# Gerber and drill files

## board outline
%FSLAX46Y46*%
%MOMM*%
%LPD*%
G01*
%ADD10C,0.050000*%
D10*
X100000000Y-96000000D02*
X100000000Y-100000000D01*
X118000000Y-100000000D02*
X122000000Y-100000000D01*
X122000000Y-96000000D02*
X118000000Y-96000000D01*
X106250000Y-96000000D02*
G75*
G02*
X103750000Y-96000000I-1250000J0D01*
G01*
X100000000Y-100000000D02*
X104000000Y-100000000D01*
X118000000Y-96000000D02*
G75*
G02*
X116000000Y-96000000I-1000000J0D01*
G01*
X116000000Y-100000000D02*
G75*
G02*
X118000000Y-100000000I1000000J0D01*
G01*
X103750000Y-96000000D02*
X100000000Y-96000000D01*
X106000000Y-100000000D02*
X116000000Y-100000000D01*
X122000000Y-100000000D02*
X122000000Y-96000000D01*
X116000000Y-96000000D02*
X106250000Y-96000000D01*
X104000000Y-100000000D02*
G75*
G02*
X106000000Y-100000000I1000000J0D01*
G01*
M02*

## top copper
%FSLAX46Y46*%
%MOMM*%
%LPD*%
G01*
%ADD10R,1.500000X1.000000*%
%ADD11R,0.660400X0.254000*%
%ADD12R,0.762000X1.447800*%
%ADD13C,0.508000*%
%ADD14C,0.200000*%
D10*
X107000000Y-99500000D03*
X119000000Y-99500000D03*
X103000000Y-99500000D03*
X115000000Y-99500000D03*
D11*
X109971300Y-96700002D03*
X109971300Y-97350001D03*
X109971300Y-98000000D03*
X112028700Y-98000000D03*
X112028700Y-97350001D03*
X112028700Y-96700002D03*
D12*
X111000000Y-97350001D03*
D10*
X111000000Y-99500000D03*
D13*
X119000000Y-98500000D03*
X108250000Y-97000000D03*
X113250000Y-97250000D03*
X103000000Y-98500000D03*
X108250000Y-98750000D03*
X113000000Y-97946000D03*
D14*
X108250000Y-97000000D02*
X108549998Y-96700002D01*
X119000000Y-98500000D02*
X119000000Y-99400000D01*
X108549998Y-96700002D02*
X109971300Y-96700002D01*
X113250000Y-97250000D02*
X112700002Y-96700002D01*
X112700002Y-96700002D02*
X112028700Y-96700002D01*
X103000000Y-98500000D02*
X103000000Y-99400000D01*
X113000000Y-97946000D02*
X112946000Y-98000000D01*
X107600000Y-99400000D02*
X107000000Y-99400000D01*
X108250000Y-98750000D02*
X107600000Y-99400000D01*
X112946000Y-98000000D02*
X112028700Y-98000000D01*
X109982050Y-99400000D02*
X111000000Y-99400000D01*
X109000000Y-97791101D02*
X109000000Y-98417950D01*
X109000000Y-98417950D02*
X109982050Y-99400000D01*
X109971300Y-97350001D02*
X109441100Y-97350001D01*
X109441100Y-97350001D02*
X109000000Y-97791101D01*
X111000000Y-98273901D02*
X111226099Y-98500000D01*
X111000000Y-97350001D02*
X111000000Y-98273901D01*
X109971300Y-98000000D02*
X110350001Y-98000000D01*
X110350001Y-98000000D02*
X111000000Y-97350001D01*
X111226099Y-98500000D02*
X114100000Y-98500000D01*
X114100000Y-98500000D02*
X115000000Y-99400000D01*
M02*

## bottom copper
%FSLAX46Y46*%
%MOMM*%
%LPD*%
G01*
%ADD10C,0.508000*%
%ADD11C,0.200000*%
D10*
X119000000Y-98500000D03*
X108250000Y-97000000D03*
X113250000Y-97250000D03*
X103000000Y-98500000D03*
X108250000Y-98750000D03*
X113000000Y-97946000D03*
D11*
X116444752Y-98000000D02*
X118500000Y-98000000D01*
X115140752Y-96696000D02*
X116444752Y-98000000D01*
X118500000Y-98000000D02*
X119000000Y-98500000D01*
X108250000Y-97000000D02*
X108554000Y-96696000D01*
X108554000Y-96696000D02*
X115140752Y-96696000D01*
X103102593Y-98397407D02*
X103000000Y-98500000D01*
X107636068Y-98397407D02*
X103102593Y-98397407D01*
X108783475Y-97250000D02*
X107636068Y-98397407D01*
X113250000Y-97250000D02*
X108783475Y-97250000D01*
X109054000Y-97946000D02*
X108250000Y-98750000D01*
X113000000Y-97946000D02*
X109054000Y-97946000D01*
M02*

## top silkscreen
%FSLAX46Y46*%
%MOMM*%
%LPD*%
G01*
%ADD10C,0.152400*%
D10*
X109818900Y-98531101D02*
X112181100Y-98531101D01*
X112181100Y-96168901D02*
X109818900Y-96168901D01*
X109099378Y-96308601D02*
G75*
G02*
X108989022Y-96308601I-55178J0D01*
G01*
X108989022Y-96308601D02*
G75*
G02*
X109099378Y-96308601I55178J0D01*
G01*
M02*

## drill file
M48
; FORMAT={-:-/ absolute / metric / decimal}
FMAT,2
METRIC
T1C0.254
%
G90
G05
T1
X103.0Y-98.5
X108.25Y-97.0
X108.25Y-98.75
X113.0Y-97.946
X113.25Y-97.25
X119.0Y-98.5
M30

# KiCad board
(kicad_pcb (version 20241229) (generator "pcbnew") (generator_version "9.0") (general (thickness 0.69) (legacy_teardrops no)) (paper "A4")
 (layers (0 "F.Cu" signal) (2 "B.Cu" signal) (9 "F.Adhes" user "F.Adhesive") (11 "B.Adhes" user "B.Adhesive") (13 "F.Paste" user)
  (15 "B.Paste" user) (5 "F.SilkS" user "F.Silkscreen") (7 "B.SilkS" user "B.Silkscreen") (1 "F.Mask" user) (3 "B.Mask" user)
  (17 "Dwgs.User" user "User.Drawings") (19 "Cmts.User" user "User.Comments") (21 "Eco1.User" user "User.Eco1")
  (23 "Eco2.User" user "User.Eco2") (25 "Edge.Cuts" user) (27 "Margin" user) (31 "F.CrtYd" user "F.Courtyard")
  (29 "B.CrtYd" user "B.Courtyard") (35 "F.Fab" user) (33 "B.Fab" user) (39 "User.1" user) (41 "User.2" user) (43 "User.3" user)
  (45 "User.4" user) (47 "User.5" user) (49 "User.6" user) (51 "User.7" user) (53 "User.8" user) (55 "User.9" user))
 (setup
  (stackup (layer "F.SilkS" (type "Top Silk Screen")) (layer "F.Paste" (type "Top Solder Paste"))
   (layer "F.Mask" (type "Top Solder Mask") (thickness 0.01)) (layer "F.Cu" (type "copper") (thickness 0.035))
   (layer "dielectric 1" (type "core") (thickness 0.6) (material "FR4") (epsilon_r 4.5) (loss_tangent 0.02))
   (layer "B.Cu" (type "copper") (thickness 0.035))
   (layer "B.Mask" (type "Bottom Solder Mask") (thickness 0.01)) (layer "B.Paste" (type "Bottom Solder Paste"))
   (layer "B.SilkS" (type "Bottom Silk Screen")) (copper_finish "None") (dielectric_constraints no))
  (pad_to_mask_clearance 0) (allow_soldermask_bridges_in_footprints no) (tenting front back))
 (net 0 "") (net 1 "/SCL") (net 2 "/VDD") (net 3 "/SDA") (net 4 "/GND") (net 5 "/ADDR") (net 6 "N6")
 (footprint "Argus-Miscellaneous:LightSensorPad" (layer "F.Cu") (at 107 100.5)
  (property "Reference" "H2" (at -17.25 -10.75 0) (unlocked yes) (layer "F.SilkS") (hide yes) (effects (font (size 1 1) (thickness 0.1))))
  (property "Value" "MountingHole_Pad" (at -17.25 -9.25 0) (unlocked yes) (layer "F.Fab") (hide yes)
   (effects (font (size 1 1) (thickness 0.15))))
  (pad "1" smd rect (at 0 -1) (size 1.5 1) (layers "F.Cu" "F.Mask" "F.Paste") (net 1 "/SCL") (thermal_bridge_angle 45)))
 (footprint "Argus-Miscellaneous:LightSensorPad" (layer "F.Cu") (at 119 100.5)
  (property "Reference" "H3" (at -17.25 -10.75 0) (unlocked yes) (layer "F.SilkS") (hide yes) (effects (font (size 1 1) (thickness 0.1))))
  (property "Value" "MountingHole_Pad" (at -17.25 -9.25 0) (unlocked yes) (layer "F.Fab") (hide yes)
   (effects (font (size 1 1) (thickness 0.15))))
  (pad "1" smd rect (at 0 -1) (size 1.5 1) (layers "F.Cu" "F.Mask" "F.Paste") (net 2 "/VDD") (thermal_bridge_angle 45)))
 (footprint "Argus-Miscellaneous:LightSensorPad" (layer "F.Cu") (at 103 100.5)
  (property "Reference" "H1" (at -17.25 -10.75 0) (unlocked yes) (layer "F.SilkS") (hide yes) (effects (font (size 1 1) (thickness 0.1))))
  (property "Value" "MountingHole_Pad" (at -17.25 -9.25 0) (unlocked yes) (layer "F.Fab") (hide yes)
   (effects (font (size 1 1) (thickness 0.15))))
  (pad "1" smd rect (at 0 -1) (size 1.5 1) (layers "F.Cu" "F.Mask" "F.Paste") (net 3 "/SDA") (thermal_bridge_angle 45)))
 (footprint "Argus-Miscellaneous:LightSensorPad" (layer "F.Cu") (at 115 100.5)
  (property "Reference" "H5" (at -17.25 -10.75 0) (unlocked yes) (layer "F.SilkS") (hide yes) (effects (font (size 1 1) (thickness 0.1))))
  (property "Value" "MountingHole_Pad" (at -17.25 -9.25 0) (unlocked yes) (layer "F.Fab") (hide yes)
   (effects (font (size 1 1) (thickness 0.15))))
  (pad "1" smd rect (at 0 -1) (size 1.5 1) (layers "F.Cu" "F.Mask" "F.Paste") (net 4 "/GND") (thermal_bridge_angle 45)))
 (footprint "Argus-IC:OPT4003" (layer "F.Cu") (at 111 97.350001)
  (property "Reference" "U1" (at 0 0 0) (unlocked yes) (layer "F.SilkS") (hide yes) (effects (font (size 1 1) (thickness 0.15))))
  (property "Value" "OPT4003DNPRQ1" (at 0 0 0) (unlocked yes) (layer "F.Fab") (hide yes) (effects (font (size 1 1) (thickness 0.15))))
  (fp_line (start -1.1811 1.1811) (end 1.1811 1.1811) (stroke (width 0.1524) (type solid)) (layer "F.SilkS"))
  (fp_line (start 1.1811 -1.1811) (end -1.1811 -1.1811) (stroke (width 0.1524) (type solid)) (layer "F.SilkS"))
  (fp_circle (center -1.9558 -1.0414) (end -1.9027 -1.0264) (stroke (width 0.1524) (type solid)) (fill no) (layer "F.SilkS"))
  (pad "1" smd rect (at -1.0287 -0.649999) (size 0.6604 0.254) (layers "F.Cu" "F.Mask" "F.Paste") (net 2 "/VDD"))
  (pad "2" smd rect (at -1.0287 0) (size 0.6604 0.254) (layers "F.Cu" "F.Mask" "F.Paste") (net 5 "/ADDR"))
  (pad "3" smd rect (at -1.0287 0.649999) (size 0.6604 0.254) (layers "F.Cu" "F.Mask" "F.Paste") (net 4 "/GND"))
  (pad "4" smd rect (at 1.0287 0.649999) (size 0.6604 0.254) (layers "F.Cu" "F.Mask" "F.Paste") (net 1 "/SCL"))
  (pad "5" smd rect (at 1.0287 0) (size 0.6604 0.254) (layers "F.Cu" "F.Mask" "F.Paste") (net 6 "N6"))
  (pad "6" smd rect (at 1.0287 -0.649999) (size 0.6604 0.254) (layers "F.Cu" "F.Mask" "F.Paste") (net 3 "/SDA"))
  (pad "7" smd rect (at 0 0) (size 0.762 1.4478) (layers "F.Cu" "F.Mask" "F.Paste") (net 4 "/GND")))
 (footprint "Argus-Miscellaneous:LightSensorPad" (layer "F.Cu") (at 111 100.5)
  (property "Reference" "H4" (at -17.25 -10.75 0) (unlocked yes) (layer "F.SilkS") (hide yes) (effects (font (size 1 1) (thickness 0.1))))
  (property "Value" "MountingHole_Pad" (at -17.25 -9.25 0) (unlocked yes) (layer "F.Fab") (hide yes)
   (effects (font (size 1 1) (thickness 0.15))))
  (pad "1" smd rect (at 0 -1) (size 1.5 1) (layers "F.Cu" "F.Mask" "F.Paste") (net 5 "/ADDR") (thermal_bridge_angle 45)))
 (gr_line (start 100 96) (end 100 100) (stroke (width 0.05) (type default)) (layer "Edge.Cuts"))
 (gr_line (start 118 100) (end 122 100) (stroke (width 0.05) (type default)) (layer "Edge.Cuts"))
 (gr_line (start 122 96) (end 118 96) (stroke (width 0.05) (type default)) (layer "Edge.Cuts"))
 (gr_arc (start 106.25 96) (mid 105 97.25) (end 103.75 96) (stroke (width 0.05) (type default)) (layer "Edge.Cuts"))
 (gr_line (start 100 100) (end 104 100) (stroke (width 0.05) (type default)) (layer "Edge.Cuts"))
 (gr_arc (start 118 96) (mid 117 97) (end 116 96) (stroke (width 0.05) (type default)) (layer "Edge.Cuts"))
 (gr_arc (start 116 100) (mid 117 99) (end 118 100) (stroke (width 0.05) (type default)) (layer "Edge.Cuts"))
 (gr_line (start 103.75 96) (end 100 96) (stroke (width 0.05) (type default)) (layer "Edge.Cuts"))
 (gr_line (start 106 100) (end 116 100) (stroke (width 0.05) (type default)) (layer "Edge.Cuts"))
 (gr_line (start 122 100) (end 122 96) (stroke (width 0.05) (type default)) (layer "Edge.Cuts"))
 (gr_line (start 116 96) (end 106.25 96) (stroke (width 0.05) (type default)) (layer "Edge.Cuts"))
 (gr_arc (start 104 100) (mid 105 99) (end 106 100) (stroke (width 0.05) (type default)) (layer "Edge.Cuts"))
 (segment (start 108.25 97) (end 108.549998 96.700002) (width 0.2) (layer "F.Cu") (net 2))
 (segment (start 119 98.5) (end 119 99.4) (width 0.2) (layer "F.Cu") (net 2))
 (segment (start 108.549998 96.700002) (end 109.9713 96.700002) (width 0.2) (layer "F.Cu") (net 2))
 (via (at 119 98.5) (size 0.508) (drill 0.254) (layers "F.Cu" "B.Cu") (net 2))
 (via (at 108.25 97) (size 0.508) (drill 0.254) (layers "F.Cu" "B.Cu") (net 2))
 (segment (start 116.444752 98) (end 118.5 98) (width 0.2) (layer "B.Cu") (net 2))
 (segment (start 115.140752 96.696) (end 116.444752 98) (width 0.2) (layer "B.Cu") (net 2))
 (segment (start 118.5 98) (end 119 98.5) (width 0.2) (layer "B.Cu") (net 2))
 (segment (start 108.25 97) (end 108.554 96.696) (width 0.2) (layer "B.Cu") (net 2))
 (segment (start 108.554 96.696) (end 115.140752 96.696) (width 0.2) (layer "B.Cu") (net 2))
 (segment (start 113.25 97.25) (end 112.700002 96.700002) (width 0.2) (layer "F.Cu") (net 3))
 (segment (start 112.700002 96.700002) (end 112.0287 96.700002) (width 0.2) (layer "F.Cu") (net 3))
 (segment (start 103 98.5) (end 103 99.4) (width 0.2) (layer "F.Cu") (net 3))
 (via (at 113.25 97.25) (size 0.508) (drill 0.254) (layers "F.Cu" "B.Cu") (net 3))
 (via (at 103 98.5) (size 0.508) (drill 0.254) (layers "F.Cu" "B.Cu") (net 3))
 (segment (start 103.102593 98.397407) (end 103 98.5) (width 0.2) (layer "B.Cu") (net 3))
 (segment (start 107.636068 98.397407) (end 103.102593 98.397407) (width 0.2) (layer "B.Cu") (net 3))
 (segment (start 108.783475 97.25) (end 107.636068 98.397407) (width 0.2) (layer "B.Cu") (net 3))
 (segment (start 113.25 97.25) (end 108.783475 97.25) (width 0.2) (layer "B.Cu") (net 3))
 (segment (start 113 97.946) (end 112.946 98) (width 0.2) (layer "F.Cu") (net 1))
 (segment (start 107.6 99.4) (end 107 99.4) (width 0.2) (layer "F.Cu") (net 1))
 (segment (start 108.25 98.75) (end 107.6 99.4) (width 0.2) (layer "F.Cu") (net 1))
 (segment (start 112.946 98) (end 112.0287 98) (width 0.2) (layer "F.Cu") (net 1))
 (via (at 108.25 98.75) (size 0.508) (drill 0.254) (layers "F.Cu" "B.Cu") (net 1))
 (via (at 113 97.946) (size 0.508) (drill 0.254) (layers "F.Cu" "B.Cu") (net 1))
 (segment (start 109.054 97.946) (end 108.25 98.75) (width 0.2) (layer "B.Cu") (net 1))
 (segment (start 113 97.946) (end 109.054 97.946) (width 0.2) (layer "B.Cu") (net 1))
 (segment (start 109.98205 99.4) (end 111 99.4) (width 0.2) (layer "F.Cu") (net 5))
 (segment (start 109 97.791101) (end 109 98.41795) (width 0.2) (layer "F.Cu") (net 5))
 (segment (start 109 98.41795) (end 109.98205 99.4) (width 0.2) (layer "F.Cu") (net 5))
 (segment (start 109.9713 97.350001) (end 109.4411 97.350001) (width 0.2) (layer "F.Cu") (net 5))
 (segment (start 109.4411 97.350001) (end 109 97.791101) (width 0.2) (layer "F.Cu") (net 5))
 (segment (start 111 98.273901) (end 111.226099 98.5) (width 0.2) (layer "F.Cu") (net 4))
 (segment (start 111 97.350001) (end 111 98.273901) (width 0.2) (layer "F.Cu") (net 4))
 (segment (start 109.9713 98) (end 110.350001 98) (width 0.2) (layer "F.Cu") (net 4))
 (segment (start 110.350001 98) (end 111 97.350001) (width 0.2) (layer "F.Cu") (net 4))
 (segment (start 111.226099 98.5) (end 114.1 98.5) (width 0.2) (layer "F.Cu") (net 4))
 (segment (start 114.1 98.5) (end 115 99.4) (width 0.2) (layer "F.Cu") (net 4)))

